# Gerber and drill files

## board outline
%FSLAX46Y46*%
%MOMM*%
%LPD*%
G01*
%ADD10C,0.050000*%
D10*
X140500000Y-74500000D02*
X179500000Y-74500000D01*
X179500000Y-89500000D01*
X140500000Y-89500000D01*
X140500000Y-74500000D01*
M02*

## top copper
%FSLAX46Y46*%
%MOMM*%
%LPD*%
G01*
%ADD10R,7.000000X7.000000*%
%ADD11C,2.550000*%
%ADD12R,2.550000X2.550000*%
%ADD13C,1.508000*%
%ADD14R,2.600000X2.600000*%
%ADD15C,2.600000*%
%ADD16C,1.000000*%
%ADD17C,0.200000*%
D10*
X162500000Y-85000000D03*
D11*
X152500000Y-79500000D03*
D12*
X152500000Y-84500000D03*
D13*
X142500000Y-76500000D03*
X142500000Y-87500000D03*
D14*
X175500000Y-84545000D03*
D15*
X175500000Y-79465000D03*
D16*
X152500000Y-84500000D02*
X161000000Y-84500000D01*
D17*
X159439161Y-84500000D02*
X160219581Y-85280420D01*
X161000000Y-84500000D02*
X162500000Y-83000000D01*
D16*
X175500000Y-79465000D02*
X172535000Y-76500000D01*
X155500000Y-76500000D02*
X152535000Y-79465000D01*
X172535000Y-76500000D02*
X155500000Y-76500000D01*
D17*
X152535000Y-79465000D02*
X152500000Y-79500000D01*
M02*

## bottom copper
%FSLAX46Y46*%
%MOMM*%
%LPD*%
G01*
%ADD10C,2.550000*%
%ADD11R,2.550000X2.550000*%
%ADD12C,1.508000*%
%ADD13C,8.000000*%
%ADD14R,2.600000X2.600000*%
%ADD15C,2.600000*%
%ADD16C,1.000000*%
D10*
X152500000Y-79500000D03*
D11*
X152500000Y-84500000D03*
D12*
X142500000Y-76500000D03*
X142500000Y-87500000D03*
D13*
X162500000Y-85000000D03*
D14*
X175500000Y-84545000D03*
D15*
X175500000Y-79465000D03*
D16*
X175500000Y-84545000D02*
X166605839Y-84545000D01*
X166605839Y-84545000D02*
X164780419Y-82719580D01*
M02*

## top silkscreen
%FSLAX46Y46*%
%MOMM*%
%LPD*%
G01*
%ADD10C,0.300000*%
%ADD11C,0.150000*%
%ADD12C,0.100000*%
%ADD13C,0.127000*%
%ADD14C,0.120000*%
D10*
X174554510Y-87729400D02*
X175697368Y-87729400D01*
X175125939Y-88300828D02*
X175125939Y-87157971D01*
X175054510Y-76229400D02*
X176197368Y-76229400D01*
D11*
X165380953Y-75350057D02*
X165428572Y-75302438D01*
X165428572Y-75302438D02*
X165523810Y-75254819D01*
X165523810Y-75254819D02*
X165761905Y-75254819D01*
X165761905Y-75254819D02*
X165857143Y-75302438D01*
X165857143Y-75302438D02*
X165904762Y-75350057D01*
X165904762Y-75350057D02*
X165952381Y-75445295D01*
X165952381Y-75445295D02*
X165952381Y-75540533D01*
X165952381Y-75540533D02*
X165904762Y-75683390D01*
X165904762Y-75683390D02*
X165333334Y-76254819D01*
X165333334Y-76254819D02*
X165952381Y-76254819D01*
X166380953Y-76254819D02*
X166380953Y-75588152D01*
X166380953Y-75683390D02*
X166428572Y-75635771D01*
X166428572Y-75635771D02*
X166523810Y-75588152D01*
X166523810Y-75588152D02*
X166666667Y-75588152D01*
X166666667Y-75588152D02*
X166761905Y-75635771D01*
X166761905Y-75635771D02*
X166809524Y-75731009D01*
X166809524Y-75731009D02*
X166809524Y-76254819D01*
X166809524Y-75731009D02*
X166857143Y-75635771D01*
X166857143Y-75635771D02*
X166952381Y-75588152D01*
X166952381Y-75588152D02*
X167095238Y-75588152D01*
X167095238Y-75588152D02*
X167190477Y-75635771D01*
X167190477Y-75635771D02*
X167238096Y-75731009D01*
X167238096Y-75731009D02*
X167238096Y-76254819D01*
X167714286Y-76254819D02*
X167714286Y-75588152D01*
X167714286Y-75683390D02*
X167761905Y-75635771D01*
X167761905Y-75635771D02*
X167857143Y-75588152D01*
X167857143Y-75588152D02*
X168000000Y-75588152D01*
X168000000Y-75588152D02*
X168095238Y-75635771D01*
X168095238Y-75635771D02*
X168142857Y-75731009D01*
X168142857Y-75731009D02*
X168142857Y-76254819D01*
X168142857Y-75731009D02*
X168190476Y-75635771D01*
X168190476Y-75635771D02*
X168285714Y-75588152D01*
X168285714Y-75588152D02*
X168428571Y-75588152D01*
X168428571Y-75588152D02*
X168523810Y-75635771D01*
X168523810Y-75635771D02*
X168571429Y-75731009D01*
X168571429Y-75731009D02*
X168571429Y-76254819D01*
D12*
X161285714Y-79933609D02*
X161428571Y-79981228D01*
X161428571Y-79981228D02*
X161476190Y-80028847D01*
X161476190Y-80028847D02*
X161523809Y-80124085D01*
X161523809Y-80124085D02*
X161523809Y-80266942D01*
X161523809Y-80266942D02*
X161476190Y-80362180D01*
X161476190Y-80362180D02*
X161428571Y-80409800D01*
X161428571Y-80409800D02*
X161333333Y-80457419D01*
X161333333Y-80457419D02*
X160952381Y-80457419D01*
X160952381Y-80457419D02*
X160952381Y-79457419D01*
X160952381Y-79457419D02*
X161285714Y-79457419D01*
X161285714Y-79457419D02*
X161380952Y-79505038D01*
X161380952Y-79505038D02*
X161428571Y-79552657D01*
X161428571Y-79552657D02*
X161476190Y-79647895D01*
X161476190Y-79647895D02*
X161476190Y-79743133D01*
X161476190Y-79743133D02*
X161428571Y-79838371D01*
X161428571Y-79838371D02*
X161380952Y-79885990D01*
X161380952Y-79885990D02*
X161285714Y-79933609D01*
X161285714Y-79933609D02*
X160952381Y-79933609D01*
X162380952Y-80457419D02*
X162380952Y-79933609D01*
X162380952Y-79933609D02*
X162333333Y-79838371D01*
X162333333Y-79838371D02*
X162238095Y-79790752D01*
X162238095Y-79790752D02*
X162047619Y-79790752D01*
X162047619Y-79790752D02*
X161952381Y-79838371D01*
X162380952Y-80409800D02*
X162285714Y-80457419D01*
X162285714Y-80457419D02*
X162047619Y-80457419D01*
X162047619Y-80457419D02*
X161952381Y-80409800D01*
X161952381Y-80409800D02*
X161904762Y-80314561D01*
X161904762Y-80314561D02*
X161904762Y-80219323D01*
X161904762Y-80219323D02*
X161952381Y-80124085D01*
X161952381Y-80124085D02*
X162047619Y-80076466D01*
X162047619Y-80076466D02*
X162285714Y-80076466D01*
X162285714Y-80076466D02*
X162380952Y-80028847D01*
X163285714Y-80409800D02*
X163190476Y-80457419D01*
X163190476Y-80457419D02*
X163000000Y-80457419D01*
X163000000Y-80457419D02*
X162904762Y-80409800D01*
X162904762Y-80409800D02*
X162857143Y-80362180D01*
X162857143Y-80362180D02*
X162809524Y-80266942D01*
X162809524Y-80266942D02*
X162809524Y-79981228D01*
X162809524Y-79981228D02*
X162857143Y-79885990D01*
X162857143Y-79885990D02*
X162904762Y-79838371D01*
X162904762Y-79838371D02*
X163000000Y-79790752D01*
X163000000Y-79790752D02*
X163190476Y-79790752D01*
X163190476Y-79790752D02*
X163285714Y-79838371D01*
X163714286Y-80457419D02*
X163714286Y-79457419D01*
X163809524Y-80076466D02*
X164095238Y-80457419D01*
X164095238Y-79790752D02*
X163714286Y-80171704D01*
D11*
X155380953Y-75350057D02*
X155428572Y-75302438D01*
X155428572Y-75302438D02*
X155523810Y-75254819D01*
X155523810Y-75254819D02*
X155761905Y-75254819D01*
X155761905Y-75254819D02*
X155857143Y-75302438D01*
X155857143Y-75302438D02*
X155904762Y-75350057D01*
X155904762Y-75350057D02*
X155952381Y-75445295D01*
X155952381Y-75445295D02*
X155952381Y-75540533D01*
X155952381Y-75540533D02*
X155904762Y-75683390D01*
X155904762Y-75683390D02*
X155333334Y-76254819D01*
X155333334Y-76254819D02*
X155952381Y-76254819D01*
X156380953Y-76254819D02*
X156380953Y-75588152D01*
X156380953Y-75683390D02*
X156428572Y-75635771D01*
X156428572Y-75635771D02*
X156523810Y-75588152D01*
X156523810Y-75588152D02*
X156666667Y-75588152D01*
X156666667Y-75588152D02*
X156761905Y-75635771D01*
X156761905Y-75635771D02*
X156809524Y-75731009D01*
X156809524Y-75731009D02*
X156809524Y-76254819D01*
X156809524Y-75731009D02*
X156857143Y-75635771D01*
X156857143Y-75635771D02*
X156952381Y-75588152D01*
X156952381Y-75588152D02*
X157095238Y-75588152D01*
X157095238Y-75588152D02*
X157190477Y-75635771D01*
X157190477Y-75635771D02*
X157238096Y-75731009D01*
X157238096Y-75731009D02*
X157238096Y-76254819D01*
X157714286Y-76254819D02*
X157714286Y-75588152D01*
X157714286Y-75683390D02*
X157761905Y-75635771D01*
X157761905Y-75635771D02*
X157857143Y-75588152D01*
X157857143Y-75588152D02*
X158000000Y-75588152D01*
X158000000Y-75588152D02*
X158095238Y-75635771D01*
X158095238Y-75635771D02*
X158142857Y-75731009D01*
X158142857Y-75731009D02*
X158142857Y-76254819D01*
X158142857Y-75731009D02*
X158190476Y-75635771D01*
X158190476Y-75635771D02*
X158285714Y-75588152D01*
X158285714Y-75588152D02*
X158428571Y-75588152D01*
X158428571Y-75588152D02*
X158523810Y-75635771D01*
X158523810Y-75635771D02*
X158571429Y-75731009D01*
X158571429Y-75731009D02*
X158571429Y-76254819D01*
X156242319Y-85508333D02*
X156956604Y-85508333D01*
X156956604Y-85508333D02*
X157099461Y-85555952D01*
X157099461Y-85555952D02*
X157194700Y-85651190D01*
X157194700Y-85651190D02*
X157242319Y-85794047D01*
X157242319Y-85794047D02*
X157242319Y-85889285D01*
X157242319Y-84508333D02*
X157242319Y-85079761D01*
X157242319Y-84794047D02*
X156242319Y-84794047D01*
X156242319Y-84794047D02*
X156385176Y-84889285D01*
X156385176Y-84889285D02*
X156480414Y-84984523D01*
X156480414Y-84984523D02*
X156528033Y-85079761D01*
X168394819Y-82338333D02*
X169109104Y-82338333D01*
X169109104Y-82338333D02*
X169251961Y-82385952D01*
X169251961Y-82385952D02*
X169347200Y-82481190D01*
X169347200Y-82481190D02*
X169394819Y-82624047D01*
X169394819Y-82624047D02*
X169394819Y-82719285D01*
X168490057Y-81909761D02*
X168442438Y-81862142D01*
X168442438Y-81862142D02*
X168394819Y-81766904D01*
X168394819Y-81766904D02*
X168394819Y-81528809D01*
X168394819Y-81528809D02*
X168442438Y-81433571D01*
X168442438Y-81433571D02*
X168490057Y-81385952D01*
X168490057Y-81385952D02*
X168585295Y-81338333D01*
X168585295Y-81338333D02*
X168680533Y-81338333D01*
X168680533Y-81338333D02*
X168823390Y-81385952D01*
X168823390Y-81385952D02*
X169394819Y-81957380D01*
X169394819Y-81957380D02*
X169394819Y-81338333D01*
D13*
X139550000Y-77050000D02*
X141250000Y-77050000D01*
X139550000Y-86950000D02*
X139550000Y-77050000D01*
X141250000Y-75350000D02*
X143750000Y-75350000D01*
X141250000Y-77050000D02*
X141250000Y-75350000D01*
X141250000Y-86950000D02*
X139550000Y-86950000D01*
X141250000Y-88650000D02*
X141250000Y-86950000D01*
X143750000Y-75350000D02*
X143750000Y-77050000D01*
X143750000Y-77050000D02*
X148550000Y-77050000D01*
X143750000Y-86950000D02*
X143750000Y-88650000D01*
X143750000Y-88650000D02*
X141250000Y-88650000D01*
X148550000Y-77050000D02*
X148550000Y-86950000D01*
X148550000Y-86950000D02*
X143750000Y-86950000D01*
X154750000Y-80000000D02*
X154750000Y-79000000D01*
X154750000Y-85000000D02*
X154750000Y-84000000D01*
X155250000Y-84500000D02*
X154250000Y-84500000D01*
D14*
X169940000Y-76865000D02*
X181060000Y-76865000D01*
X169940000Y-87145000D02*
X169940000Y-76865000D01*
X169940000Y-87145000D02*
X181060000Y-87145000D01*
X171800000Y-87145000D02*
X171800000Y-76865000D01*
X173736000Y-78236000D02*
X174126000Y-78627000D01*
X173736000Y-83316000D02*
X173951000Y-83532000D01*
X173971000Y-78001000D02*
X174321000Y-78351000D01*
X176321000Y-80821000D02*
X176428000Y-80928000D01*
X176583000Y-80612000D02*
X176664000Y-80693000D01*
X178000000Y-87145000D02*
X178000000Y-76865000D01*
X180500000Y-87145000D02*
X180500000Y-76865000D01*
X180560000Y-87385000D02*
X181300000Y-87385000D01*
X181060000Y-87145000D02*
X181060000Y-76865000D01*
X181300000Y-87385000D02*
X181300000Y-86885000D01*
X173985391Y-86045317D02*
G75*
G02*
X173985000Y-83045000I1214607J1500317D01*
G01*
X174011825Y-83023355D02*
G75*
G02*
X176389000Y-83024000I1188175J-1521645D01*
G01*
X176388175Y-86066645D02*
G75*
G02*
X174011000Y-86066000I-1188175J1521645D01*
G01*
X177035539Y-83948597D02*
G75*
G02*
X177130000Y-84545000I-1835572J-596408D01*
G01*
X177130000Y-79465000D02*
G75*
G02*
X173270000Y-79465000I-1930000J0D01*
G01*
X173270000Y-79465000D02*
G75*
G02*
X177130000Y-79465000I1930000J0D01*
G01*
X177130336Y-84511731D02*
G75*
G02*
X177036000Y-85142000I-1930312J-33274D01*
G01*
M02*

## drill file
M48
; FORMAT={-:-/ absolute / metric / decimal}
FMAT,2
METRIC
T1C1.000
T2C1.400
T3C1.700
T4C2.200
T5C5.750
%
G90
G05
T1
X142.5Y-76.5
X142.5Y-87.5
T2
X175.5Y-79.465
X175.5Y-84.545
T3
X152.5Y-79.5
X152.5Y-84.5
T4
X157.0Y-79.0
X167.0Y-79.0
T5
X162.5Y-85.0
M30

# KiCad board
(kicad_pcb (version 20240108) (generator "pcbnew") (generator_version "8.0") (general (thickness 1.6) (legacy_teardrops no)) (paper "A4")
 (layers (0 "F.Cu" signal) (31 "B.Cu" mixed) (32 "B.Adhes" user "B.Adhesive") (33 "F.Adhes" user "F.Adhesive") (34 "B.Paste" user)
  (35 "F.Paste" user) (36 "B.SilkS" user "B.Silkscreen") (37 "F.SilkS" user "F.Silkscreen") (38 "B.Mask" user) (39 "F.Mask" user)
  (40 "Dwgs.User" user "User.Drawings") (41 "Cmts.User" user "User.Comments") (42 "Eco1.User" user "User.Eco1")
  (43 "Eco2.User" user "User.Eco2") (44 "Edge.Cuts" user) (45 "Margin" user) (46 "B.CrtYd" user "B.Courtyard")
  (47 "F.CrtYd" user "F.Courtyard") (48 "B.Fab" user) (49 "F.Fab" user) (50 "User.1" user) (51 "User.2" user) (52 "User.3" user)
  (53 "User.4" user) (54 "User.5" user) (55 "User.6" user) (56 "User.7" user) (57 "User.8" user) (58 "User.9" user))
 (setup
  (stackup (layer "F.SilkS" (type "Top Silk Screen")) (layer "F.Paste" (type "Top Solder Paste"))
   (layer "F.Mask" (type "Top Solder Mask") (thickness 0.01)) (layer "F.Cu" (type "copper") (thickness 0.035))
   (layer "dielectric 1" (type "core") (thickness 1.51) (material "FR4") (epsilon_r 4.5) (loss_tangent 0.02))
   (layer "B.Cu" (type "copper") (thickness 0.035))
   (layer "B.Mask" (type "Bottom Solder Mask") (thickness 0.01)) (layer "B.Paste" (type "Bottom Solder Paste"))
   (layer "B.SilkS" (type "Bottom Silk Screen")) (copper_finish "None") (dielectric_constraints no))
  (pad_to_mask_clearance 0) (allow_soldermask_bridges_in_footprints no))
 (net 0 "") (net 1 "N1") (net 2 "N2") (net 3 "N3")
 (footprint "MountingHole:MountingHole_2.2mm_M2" (layer "F.Cu") (at 167 79)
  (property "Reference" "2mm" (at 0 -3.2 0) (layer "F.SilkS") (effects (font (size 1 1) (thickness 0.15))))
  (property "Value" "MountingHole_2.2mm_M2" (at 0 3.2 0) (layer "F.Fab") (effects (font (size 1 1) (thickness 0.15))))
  (pad "" np_thru_hole circle (at 0 0) (size 2.2 2.2) (drill 2.2) (layers "*.Cu" "*.Mask")))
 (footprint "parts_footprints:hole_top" (layer "F.Cu") (at 162.5 85)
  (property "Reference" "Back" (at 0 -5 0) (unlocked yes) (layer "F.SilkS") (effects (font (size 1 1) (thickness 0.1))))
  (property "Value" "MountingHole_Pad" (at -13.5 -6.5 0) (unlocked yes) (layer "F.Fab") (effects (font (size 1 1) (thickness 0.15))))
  (pad "1" smd rect (at 0 0) (size 7 7) (layers "F.Cu" "F.Paste" "F.Mask") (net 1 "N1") (solder_mask_margin 0.102)))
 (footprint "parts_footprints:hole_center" (layer "F.Cu") (at 162.5 85)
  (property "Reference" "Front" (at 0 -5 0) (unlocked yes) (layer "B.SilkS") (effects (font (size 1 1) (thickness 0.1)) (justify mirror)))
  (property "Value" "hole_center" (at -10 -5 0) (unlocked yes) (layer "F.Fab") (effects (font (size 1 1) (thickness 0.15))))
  (pad "" np_thru_hole circle (at 0 0) (size 1.524 1.524) (drill 5.75) (layers "*.Mask")))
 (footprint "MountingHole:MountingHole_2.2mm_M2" (layer "F.Cu") (at 157 79)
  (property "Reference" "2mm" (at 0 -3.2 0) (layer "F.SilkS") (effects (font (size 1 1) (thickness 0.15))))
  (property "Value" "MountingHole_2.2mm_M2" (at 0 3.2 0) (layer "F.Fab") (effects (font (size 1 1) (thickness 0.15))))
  (pad "" np_thru_hole circle (at 0 0) (size 2.2 2.2) (drill 2.2) (layers "*.Cu" "*.Mask")))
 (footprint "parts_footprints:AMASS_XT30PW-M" (layer "F.Cu") (at 142.5 82 90)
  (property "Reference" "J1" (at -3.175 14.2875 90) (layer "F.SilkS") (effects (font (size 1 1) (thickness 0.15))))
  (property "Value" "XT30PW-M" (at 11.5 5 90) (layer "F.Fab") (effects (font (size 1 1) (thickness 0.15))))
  (fp_line (start 4.95 -2.95) (end 4.95 -1.25) (stroke (width 0.127) (type solid)) (layer "F.SilkS"))
  (fp_line (start -4.95 -2.95) (end 4.95 -2.95) (stroke (width 0.127) (type solid)) (layer "F.SilkS"))
  (fp_line (start 6.65 -1.25) (end 6.65 1.25) (stroke (width 0.127) (type solid)) (layer "F.SilkS"))
  (fp_line (start 4.95 -1.25) (end 6.65 -1.25) (stroke (width 0.127) (type solid)) (layer "F.SilkS"))
  (fp_line (start -4.95 -1.25) (end -4.95 -2.95) (stroke (width 0.127) (type solid)) (layer "F.SilkS"))
  (fp_line (start -6.65 -1.25) (end -4.95 -1.25) (stroke (width 0.127) (type solid)) (layer "F.SilkS"))
  (fp_line (start 6.65 1.25) (end 4.95 1.25) (stroke (width 0.127) (type solid)) (layer "F.SilkS"))
  (fp_line (start 4.95 1.25) (end 4.95 6.05) (stroke (width 0.127) (type solid)) (layer "F.SilkS"))
  (fp_line (start -4.95 1.25) (end -6.65 1.25) (stroke (width 0.127) (type solid)) (layer "F.SilkS"))
  (fp_line (start -6.65 1.25) (end -6.65 -1.25) (stroke (width 0.127) (type solid)) (layer "F.SilkS"))
  (fp_line (start 4.95 6.05) (end -4.95 6.05) (stroke (width 0.127) (type solid)) (layer "F.SilkS"))
  (fp_line (start -4.95 6.05) (end -4.95 1.25) (stroke (width 0.127) (type solid)) (layer "F.SilkS"))
  (fp_line (start 2 12.25) (end 3 12.25) (stroke (width 0.127) (type solid)) (layer "F.SilkS"))
  (fp_line (start -3 12.25) (end -2 12.25) (stroke (width 0.127) (type solid)) (layer "F.SilkS"))
  (fp_line (start -2.5 12.75) (end -2.5 11.75) (stroke (width 0.127) (type solid)) (layer "F.SilkS"))
  (pad "N" thru_hole circle (at 2.5 10 90) (size 2.55 2.55) (drill 1.7) (layers "*.Cu" "*.Mask") (remove_unused_layers no) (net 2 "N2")
   (solder_mask_margin 0.102))
  (pad "P" thru_hole rect (at -2.5 10 90) (size 2.55 2.55) (drill 1.7) (layers "*.Cu" "*.Mask") (remove_unused_layers no) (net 1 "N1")
   (solder_mask_margin 0.102))
  (pad "S1" thru_hole circle (at 5.5 0 90) (size 1.508 1.508) (drill 1) (layers "*.Cu" "*.Mask") (remove_unused_layers no)
   (solder_mask_margin 0.102))
  (pad "S2" thru_hole circle (at -5.5 0 90) (size 1.508 1.508) (drill 1) (layers "*.Cu" "*.Mask") (remove_unused_layers no)
   (solder_mask_margin 0.102)))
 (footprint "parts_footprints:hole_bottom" (layer "F.Cu") (at 162.5 85)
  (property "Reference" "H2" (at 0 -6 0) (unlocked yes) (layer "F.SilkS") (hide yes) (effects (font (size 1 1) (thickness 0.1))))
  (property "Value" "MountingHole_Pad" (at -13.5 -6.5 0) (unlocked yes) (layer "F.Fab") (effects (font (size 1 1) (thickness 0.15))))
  (pad "1" smd circle (at 0 0) (size 8 8) (layers "B.Cu" "B.Paste" "B.Mask") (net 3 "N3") (solder_mask_margin 0.102)))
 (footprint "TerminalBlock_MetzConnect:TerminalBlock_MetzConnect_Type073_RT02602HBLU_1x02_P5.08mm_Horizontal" (layer "F.Cu")
  (at 175.5 84.545 90)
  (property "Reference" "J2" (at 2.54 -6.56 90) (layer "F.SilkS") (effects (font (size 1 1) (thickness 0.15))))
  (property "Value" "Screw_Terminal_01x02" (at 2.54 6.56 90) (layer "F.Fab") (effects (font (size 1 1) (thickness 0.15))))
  (fp_line (start 7.68 -5.56) (end 7.68 5.56) (stroke (width 0.12) (type solid)) (layer "F.SilkS"))
  (fp_line (start -2.6 -5.56) (end 7.68 -5.56) (stroke (width 0.12) (type solid)) (layer "F.SilkS"))
  (fp_line (start -2.6 -5.56) (end -2.6 5.56) (stroke (width 0.12) (type solid)) (layer "F.SilkS"))
  (fp_line (start -2.6 -3.7) (end 7.68 -3.7) (stroke (width 0.12) (type solid)) (layer "F.SilkS"))
  (fp_line (start 6.309 -1.764) (end 5.918 -1.374) (stroke (width 0.12) (type solid)) (layer "F.SilkS"))
  (fp_line (start 1.229 -1.764) (end 1.013 -1.549) (stroke (width 0.12) (type solid)) (layer "F.SilkS"))
  (fp_line (start 6.544 -1.529) (end 6.194 -1.179) (stroke (width 0.12) (type solid)) (layer "F.SilkS"))
  (fp_line (start 3.724 0.821) (end 3.617 0.928) (stroke (width 0.12) (type solid)) (layer "F.SilkS"))
  (fp_line (start 3.933 1.083) (end 3.852 1.164) (stroke (width 0.12) (type solid)) (layer "F.SilkS"))
  (fp_line (start -2.6 2.5) (end 7.68 2.5) (stroke (width 0.12) (type solid)) (layer "F.SilkS"))
  (fp_line (start -2.6 5) (end 7.68 5) (stroke (width 0.12) (type solid)) (layer "F.SilkS"))
  (fp_line (start -2.84 5.06) (end -2.84 5.8) (stroke (width 0.12) (type solid)) (layer "F.SilkS"))
  (fp_line (start -2.6 5.56) (end 7.68 5.56) (stroke (width 0.12) (type solid)) (layer "F.SilkS"))
  (fp_line (start -2.84 5.8) (end -2.34 5.8) (stroke (width 0.12) (type solid)) (layer "F.SilkS"))
  (fp_arc (start -1.500317 -1.514609) (mid -0.000252 -2.230344) (end 1.5 -1.515) (stroke (width 0.12) (type solid)) (layer "F.SilkS"))
  (fp_arc (start 1.521645 -1.488175) (mid 1.930586 -0.299476) (end 1.521 0.889) (stroke (width 0.12) (type solid)) (layer "F.SilkS"))
  (fp_arc (start -1.521645 0.888175) (mid -1.930586 -0.300524) (end -1.521 -1.489) (stroke (width 0.12) (type solid)) (layer "F.SilkS"))
  (fp_arc (start 0.596403 1.535539) (mid 0.301919 1.606238) (end 0 1.63) (stroke (width 0.12) (type solid)) (layer "F.SilkS"))
  (fp_arc (start 5.08 1.63) (mid 5.08 -2.23) (end 5.08 1.63) (stroke (width 0.12) (type solid)) (layer "F.SilkS"))
  (fp_arc (start 0.033269 1.630336) (mid -0.285785 1.609354) (end -0.597 1.536) (stroke (width 0.12) (type solid)) (layer "F.SilkS"))
  (pad "1" thru_hole rect (at 0 0 90) (size 2.6 2.6) (drill 1.4) (layers "*.Cu" "*.Mask") (remove_unused_layers no) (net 3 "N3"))
  (pad "2" thru_hole circle (at 5.08 0 90) (size 2.6 2.6) (drill 1.4) (layers "*.Cu" "*.Mask") (remove_unused_layers no) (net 2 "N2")))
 (gr_rect (start 140.5 74.5) (end 179.5 89.5) (stroke (width 0.05) (type default)) (fill none) (layer "Edge.Cuts"))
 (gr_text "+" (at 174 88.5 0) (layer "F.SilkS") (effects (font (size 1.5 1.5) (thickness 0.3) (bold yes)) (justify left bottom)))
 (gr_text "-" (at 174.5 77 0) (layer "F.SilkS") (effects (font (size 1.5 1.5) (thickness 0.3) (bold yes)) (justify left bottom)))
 (segment (start 152.5 84.5) (end 161 84.5) (width 1) (layer "F.Cu") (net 1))
 (segment (start 159.439161 84.5) (end 160.219581 85.28042) (width 0.2) (layer "F.Cu") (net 1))
 (segment (start 161 84.5) (end 162.5 83) (width 0.2) (layer "F.Cu") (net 1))
 (segment (start 175.5 79.465) (end 172.535 76.5) (width 1) (layer "F.Cu") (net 2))
 (segment (start 155.5 76.5) (end 152.535 79.465) (width 1) (layer "F.Cu") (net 2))
 (segment (start 172.535 76.5) (end 155.5 76.5) (width 1) (layer "F.Cu") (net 2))
 (segment (start 152.535 79.465) (end 152.5 79.5) (width 0.2) (layer "F.Cu") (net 2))
 (segment (start 175.5 84.545) (end 166.605839 84.545) (width 1) (layer "B.Cu") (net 3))
 (segment (start 166.605839 84.545) (end 164.780419 82.71958) (width 1) (layer "B.Cu") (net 3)))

